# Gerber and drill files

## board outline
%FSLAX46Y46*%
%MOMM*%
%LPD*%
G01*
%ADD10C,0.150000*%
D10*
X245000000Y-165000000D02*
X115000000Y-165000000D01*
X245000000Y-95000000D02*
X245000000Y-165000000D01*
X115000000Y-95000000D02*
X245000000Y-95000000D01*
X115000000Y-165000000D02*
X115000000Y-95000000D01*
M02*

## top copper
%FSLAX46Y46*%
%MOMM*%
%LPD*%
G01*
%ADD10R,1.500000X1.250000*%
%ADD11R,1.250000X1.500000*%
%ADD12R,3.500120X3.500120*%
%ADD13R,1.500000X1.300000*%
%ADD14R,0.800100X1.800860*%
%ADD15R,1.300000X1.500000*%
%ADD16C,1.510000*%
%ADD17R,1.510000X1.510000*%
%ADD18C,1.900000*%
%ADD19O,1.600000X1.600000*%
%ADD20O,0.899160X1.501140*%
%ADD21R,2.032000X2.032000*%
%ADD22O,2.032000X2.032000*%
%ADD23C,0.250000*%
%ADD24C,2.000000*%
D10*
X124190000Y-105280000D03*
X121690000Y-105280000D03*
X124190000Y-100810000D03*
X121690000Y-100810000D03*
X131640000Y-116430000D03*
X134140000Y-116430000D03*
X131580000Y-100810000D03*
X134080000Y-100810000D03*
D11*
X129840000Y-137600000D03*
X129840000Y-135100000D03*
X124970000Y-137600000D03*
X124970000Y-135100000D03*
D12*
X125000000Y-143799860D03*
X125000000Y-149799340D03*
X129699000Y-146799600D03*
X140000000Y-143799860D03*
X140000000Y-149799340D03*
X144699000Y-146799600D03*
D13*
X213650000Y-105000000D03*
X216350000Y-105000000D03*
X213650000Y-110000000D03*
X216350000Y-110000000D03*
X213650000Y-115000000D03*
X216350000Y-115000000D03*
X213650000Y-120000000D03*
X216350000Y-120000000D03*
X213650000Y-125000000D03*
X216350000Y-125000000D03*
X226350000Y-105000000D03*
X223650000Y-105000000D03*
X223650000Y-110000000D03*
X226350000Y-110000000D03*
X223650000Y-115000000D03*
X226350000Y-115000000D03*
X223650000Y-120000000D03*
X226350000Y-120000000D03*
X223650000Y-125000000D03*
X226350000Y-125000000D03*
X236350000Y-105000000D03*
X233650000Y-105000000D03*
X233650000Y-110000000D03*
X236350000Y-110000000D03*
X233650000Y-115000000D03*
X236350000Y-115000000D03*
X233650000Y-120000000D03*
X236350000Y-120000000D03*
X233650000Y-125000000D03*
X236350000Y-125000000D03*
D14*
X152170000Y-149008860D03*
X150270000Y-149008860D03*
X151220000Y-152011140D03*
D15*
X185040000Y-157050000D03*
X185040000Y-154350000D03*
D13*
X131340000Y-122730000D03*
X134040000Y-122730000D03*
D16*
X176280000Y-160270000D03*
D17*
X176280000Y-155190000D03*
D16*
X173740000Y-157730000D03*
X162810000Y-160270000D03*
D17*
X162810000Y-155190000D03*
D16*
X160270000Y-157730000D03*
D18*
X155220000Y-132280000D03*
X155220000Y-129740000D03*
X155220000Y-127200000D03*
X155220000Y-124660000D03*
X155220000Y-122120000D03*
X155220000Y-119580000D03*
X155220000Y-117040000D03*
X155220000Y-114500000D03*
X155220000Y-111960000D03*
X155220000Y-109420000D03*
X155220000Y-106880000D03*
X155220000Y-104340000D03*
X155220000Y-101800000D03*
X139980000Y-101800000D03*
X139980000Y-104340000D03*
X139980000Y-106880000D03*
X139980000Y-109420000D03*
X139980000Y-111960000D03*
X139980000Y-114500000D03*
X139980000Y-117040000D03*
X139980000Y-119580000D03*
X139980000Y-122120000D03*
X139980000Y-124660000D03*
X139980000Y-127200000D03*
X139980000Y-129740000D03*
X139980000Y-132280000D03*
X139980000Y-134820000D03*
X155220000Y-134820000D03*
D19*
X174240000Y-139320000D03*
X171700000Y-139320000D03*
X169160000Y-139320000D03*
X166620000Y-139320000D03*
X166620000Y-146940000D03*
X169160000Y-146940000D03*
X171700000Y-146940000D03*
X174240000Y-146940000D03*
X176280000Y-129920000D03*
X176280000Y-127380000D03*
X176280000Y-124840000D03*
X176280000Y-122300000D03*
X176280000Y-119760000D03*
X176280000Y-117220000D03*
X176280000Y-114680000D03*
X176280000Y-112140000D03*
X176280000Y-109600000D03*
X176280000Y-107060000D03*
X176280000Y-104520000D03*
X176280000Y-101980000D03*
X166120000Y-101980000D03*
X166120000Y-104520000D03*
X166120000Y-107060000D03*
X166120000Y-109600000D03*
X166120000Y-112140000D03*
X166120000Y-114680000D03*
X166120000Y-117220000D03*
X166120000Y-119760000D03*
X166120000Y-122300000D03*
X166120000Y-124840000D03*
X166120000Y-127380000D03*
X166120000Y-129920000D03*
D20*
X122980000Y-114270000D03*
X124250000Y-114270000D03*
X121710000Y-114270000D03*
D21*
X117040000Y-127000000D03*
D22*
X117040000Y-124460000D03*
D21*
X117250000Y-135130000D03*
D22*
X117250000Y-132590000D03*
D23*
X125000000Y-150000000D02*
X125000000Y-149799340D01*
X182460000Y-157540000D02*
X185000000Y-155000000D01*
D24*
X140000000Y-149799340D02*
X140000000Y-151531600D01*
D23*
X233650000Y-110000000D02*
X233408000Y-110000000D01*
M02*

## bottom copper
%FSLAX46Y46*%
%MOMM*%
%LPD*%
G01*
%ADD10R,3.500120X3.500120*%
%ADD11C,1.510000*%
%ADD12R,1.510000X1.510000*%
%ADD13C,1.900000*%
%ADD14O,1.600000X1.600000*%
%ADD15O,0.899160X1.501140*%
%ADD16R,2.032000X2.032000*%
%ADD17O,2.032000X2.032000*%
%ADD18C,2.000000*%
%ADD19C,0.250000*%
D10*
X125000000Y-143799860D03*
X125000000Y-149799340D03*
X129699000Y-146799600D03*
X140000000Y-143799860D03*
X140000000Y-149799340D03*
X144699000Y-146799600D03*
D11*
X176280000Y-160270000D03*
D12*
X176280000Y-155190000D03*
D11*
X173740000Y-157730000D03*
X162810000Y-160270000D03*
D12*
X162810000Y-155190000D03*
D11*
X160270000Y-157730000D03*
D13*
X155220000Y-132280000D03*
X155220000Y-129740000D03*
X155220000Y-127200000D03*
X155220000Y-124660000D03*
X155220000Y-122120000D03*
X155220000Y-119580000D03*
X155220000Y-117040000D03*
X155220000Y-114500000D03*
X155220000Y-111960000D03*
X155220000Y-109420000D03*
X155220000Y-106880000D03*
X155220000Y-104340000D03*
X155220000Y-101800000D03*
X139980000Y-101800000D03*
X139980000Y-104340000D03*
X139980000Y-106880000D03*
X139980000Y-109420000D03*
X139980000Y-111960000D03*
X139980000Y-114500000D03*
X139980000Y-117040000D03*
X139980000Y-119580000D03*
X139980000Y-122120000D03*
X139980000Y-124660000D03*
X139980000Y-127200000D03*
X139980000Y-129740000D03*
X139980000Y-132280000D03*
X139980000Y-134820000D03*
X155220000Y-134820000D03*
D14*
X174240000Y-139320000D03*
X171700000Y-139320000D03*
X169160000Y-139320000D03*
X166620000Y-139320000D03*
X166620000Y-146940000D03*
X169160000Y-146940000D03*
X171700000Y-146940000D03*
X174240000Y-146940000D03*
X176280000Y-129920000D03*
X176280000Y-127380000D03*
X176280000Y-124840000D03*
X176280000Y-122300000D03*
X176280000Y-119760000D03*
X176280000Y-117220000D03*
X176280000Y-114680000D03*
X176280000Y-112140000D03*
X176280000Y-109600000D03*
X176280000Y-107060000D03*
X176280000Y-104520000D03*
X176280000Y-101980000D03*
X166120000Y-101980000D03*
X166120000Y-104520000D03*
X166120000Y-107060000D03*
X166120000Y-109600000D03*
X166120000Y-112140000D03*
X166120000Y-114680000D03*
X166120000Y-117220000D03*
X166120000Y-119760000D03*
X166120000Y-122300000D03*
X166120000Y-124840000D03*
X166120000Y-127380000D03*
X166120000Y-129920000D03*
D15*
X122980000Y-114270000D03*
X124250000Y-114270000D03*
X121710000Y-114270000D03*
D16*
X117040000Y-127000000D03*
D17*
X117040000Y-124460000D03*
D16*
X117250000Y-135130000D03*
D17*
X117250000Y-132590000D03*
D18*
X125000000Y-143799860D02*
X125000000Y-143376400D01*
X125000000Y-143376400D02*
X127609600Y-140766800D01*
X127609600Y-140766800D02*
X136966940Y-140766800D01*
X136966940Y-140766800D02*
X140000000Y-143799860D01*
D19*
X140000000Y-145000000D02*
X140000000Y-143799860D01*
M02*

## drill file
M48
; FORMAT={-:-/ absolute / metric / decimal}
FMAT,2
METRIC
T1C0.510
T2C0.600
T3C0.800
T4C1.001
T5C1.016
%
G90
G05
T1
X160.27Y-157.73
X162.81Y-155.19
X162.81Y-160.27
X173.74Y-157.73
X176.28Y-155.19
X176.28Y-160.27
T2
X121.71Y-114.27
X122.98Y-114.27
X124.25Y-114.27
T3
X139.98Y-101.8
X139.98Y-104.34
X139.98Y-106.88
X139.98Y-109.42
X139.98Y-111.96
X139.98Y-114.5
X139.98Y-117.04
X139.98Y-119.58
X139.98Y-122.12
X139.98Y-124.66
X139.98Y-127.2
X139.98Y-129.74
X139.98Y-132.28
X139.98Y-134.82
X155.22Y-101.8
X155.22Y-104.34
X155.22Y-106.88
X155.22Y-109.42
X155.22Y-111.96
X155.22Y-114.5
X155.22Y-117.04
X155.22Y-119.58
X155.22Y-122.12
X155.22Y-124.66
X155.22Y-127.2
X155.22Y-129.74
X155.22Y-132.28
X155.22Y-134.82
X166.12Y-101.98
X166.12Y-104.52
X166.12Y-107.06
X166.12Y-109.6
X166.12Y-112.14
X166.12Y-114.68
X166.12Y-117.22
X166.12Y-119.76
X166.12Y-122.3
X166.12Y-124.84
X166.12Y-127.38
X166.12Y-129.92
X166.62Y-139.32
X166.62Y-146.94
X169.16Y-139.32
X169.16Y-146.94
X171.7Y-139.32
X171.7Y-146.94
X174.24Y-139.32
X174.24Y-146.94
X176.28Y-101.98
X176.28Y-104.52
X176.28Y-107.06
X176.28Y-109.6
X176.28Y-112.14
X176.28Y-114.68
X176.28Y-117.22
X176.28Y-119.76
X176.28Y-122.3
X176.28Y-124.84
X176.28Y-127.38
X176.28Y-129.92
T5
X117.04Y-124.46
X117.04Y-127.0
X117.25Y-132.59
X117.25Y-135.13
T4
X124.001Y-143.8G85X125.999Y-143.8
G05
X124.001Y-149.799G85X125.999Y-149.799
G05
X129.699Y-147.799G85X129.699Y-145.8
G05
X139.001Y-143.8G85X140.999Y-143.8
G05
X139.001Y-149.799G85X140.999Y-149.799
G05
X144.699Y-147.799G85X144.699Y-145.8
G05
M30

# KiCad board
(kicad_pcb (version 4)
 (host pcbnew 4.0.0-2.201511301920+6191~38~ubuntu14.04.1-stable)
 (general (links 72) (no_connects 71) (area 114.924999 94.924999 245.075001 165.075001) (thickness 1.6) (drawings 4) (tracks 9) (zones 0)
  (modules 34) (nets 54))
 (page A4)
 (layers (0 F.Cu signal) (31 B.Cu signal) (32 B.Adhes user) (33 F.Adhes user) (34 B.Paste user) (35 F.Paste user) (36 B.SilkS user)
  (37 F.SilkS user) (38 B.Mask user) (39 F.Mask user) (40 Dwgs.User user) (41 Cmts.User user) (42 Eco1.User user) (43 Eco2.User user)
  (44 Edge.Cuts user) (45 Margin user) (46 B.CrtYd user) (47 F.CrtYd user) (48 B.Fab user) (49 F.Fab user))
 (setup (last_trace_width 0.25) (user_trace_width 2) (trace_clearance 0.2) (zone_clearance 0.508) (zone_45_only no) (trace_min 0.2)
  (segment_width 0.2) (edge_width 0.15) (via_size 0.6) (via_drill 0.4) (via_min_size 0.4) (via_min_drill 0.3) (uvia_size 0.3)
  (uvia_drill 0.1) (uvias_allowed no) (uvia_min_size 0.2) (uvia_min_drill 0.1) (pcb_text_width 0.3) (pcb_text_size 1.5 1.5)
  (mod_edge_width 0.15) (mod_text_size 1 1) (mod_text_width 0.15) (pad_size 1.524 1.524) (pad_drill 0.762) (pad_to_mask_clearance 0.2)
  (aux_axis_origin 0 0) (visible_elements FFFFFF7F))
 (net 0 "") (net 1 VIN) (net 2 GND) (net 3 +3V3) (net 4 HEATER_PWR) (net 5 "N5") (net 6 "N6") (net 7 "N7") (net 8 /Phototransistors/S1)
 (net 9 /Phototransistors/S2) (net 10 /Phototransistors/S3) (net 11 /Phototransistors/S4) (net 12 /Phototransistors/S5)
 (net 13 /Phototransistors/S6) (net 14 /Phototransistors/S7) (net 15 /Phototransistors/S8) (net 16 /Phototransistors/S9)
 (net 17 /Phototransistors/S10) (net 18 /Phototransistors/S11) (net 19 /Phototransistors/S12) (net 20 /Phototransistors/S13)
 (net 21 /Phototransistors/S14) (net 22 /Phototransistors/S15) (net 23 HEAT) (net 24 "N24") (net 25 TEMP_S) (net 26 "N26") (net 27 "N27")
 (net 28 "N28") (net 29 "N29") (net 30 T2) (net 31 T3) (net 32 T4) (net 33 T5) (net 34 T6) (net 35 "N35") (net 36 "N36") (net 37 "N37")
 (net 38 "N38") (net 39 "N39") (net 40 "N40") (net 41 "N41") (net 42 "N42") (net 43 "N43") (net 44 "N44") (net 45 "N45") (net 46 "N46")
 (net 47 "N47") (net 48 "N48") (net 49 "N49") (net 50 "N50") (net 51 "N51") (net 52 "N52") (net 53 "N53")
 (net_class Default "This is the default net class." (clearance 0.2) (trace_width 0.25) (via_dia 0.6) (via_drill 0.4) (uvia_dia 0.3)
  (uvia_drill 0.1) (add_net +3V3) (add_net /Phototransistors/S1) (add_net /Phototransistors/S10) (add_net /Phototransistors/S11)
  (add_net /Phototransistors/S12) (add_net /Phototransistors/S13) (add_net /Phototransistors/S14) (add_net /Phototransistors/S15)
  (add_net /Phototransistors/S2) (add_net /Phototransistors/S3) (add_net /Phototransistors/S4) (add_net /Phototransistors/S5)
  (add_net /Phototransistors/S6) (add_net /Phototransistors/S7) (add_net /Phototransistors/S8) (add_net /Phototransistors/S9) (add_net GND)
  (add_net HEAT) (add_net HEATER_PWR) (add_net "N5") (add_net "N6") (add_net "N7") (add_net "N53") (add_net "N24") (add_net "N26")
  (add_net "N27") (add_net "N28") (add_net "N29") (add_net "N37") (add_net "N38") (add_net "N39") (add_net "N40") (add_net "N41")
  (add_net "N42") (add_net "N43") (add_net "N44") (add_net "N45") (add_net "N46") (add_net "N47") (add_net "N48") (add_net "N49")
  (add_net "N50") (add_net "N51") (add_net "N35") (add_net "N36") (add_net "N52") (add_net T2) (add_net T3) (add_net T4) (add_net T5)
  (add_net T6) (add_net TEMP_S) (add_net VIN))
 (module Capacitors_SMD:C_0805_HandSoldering (layer F.Cu) (at 122.94 105.28 180)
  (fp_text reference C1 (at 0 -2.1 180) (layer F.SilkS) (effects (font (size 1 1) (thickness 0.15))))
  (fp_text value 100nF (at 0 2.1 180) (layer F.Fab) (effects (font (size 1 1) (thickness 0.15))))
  (pad 1 smd rect (at -1.25 0 180) (size 1.5 1.25) (layers F.Cu F.Paste F.Mask) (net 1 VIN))
  (pad 2 smd rect (at 1.25 0 180) (size 1.5 1.25) (layers F.Cu F.Paste F.Mask) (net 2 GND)))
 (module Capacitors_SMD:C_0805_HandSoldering (layer F.Cu) (at 122.94 100.81 180)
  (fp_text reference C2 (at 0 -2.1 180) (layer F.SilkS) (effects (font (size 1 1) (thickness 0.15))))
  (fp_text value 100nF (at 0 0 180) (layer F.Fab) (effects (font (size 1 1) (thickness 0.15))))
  (pad 1 smd rect (at -1.25 0 180) (size 1.5 1.25) (layers F.Cu F.Paste F.Mask) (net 1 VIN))
  (pad 2 smd rect (at 1.25 0 180) (size 1.5 1.25) (layers F.Cu F.Paste F.Mask) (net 2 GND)))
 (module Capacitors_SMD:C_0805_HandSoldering (layer F.Cu) (at 132.89 116.43)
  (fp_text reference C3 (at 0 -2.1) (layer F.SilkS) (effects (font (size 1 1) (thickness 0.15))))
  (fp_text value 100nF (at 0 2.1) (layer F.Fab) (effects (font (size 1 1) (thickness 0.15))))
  (pad 1 smd rect (at -1.25 0) (size 1.5 1.25) (layers F.Cu F.Paste F.Mask) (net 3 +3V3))
  (pad 2 smd rect (at 1.25 0) (size 1.5 1.25) (layers F.Cu F.Paste F.Mask) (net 2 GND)))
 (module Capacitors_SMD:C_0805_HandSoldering (layer F.Cu) (at 132.83 100.81)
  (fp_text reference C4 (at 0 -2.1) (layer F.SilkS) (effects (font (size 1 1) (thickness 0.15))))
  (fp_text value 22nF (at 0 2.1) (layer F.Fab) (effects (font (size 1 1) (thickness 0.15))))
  (pad 1 smd rect (at -1.25 0) (size 1.5 1.25) (layers F.Cu F.Paste F.Mask) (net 3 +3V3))
  (pad 2 smd rect (at 1.25 0) (size 1.5 1.25) (layers F.Cu F.Paste F.Mask) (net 2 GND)))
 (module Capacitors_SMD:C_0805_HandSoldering (layer F.Cu) (at 129.84 136.35 90)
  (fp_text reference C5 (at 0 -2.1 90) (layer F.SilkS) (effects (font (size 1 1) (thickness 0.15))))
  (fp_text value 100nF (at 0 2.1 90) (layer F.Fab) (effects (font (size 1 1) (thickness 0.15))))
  (pad 1 smd rect (at -1.25 0 90) (size 1.5 1.25) (layers F.Cu F.Paste F.Mask) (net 3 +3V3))
  (pad 2 smd rect (at 1.25 0 90) (size 1.5 1.25) (layers F.Cu F.Paste F.Mask) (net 2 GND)))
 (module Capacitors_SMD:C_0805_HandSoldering (layer F.Cu) (at 124.97 136.35 90)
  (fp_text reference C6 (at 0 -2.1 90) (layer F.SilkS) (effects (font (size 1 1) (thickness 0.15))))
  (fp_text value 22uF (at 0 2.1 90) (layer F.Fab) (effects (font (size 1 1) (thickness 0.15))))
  (pad 1 smd rect (at -1.25 0 90) (size 1.5 1.25) (layers F.Cu F.Paste F.Mask) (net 3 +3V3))
  (pad 2 smd rect (at 1.25 0 90) (size 1.5 1.25) (layers F.Cu F.Paste F.Mask) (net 2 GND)))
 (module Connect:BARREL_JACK (layer F.Cu) (at 125 150 90)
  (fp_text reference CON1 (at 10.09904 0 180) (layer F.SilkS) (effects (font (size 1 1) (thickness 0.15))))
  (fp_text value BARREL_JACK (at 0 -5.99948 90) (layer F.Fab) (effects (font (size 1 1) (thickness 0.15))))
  (pad 1 thru_hole rect (at 6.20014 0 90) (size 3.50012 3.50012) (drill oval 1.00076 2.99974) (layers *.Cu *.Mask F.SilkS)
   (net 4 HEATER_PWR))
  (pad 2 thru_hole rect (at 0.20066 0 90) (size 3.50012 3.50012) (drill oval 1.00076 2.99974) (layers *.Cu *.Mask F.SilkS) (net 2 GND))
  (pad 3 thru_hole rect (at 3.2004 4.699 90) (size 3.50012 3.50012) (drill oval 2.99974 1.00076) (layers *.Cu *.Mask F.SilkS) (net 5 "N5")))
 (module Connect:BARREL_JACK (layer F.Cu) (at 140 150 90)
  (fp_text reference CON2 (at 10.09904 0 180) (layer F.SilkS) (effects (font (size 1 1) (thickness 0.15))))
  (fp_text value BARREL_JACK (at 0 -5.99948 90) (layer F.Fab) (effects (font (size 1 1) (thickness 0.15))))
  (pad 1 thru_hole rect (at 6.20014 0 90) (size 3.50012 3.50012) (drill oval 1.00076 2.99974) (layers *.Cu *.Mask F.SilkS)
   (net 4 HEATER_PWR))
  (pad 2 thru_hole rect (at 0.20066 0 90) (size 3.50012 3.50012) (drill oval 1.00076 2.99974) (layers *.Cu *.Mask F.SilkS) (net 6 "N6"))
  (pad 3 thru_hole rect (at 3.2004 4.699 90) (size 3.50012 3.50012) (drill oval 2.99974 1.00076) (layers *.Cu *.Mask F.SilkS) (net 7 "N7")))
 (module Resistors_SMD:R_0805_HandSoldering (layer F.Cu) (at 215 105)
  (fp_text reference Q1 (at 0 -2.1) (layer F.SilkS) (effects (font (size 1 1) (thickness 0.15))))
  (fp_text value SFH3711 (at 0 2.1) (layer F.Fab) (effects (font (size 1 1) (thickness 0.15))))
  (pad 1 smd rect (at -1.35 0) (size 1.5 1.3) (layers F.Cu F.Paste F.Mask) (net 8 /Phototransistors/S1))
  (pad 2 smd rect (at 1.35 0) (size 1.5 1.3) (layers F.Cu F.Paste F.Mask) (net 3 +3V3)))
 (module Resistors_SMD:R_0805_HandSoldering (layer F.Cu) (at 215 110)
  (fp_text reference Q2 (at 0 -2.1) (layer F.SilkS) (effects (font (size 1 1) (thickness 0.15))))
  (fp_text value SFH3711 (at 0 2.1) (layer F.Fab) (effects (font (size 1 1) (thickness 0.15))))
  (pad 1 smd rect (at -1.35 0) (size 1.5 1.3) (layers F.Cu F.Paste F.Mask) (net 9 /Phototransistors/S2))
  (pad 2 smd rect (at 1.35 0) (size 1.5 1.3) (layers F.Cu F.Paste F.Mask) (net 3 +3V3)))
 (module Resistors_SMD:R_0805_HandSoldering (layer F.Cu) (at 215 115)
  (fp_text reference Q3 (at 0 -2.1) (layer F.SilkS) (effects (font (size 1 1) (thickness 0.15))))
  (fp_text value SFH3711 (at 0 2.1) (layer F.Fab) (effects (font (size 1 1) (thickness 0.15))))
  (pad 1 smd rect (at -1.35 0) (size 1.5 1.3) (layers F.Cu F.Paste F.Mask) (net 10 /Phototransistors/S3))
  (pad 2 smd rect (at 1.35 0) (size 1.5 1.3) (layers F.Cu F.Paste F.Mask) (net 3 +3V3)))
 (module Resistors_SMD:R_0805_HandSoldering (layer F.Cu) (at 215 120)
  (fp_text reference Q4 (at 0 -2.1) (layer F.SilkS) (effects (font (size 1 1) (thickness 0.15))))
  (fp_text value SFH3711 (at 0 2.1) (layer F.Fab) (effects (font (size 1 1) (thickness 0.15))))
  (pad 1 smd rect (at -1.35 0) (size 1.5 1.3) (layers F.Cu F.Paste F.Mask) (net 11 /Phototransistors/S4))
  (pad 2 smd rect (at 1.35 0) (size 1.5 1.3) (layers F.Cu F.Paste F.Mask) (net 3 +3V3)))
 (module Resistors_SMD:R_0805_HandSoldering (layer F.Cu) (at 215 125)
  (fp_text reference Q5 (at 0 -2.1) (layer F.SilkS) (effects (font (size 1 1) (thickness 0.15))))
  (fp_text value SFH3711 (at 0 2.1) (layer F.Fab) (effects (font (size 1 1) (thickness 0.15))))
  (pad 1 smd rect (at -1.35 0) (size 1.5 1.3) (layers F.Cu F.Paste F.Mask) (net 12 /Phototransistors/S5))
  (pad 2 smd rect (at 1.35 0) (size 1.5 1.3) (layers F.Cu F.Paste F.Mask) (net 3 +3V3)))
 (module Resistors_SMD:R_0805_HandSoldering (layer F.Cu) (at 225 105 180)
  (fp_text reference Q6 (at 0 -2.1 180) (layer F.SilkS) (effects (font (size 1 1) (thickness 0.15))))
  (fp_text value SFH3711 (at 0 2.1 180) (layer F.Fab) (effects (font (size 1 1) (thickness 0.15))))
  (pad 1 smd rect (at -1.35 0 180) (size 1.5 1.3) (layers F.Cu F.Paste F.Mask) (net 3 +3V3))
  (pad 2 smd rect (at 1.35 0 180) (size 1.5 1.3) (layers F.Cu F.Paste F.Mask) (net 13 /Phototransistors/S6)))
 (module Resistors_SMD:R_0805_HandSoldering (layer F.Cu) (at 225 110)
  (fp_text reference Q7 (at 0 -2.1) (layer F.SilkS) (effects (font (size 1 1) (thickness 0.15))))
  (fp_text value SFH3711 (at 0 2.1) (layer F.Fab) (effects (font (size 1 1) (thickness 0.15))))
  (pad 1 smd rect (at -1.35 0) (size 1.5 1.3) (layers F.Cu F.Paste F.Mask) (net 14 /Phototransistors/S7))
  (pad 2 smd rect (at 1.35 0) (size 1.5 1.3) (layers F.Cu F.Paste F.Mask) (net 3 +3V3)))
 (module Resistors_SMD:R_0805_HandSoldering (layer F.Cu) (at 225 115)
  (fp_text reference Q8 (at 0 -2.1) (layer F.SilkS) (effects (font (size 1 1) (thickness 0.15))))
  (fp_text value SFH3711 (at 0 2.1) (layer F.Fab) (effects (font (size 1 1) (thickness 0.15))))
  (pad 1 smd rect (at -1.35 0) (size 1.5 1.3) (layers F.Cu F.Paste F.Mask) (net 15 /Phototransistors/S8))
  (pad 2 smd rect (at 1.35 0) (size 1.5 1.3) (layers F.Cu F.Paste F.Mask) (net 3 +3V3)))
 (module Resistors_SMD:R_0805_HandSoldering (layer F.Cu) (at 225 120)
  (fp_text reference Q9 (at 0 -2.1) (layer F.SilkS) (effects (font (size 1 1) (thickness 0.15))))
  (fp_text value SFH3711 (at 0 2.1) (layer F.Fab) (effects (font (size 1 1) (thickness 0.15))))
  (pad 1 smd rect (at -1.35 0) (size 1.5 1.3) (layers F.Cu F.Paste F.Mask) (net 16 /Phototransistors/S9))
  (pad 2 smd rect (at 1.35 0) (size 1.5 1.3) (layers F.Cu F.Paste F.Mask) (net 3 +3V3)))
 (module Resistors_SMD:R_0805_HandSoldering (layer F.Cu) (at 225 125)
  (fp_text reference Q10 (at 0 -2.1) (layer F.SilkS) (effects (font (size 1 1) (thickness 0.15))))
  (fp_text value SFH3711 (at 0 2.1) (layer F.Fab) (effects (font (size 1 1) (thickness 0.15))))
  (pad 1 smd rect (at -1.35 0) (size 1.5 1.3) (layers F.Cu F.Paste F.Mask) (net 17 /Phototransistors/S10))
  (pad 2 smd rect (at 1.35 0) (size 1.5 1.3) (layers F.Cu F.Paste F.Mask) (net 3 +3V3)))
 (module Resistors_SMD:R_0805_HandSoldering (layer F.Cu) (at 235 105 180)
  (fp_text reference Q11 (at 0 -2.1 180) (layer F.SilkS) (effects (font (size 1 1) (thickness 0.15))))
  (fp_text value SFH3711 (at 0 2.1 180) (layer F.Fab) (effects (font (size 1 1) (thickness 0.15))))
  (pad 1 smd rect (at -1.35 0 180) (size 1.5 1.3) (layers F.Cu F.Paste F.Mask) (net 3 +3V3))
  (pad 2 smd rect (at 1.35 0 180) (size 1.5 1.3) (layers F.Cu F.Paste F.Mask) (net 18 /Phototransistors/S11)))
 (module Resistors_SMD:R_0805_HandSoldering (layer F.Cu) (at 235 110)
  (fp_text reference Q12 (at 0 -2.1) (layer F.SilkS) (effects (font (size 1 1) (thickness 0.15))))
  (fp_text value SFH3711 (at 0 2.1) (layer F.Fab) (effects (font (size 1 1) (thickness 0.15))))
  (pad 1 smd rect (at -1.35 0) (size 1.5 1.3) (layers F.Cu F.Paste F.Mask) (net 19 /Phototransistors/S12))
  (pad 2 smd rect (at 1.35 0) (size 1.5 1.3) (layers F.Cu F.Paste F.Mask) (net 3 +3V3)))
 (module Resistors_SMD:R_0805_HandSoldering (layer F.Cu) (at 235 115)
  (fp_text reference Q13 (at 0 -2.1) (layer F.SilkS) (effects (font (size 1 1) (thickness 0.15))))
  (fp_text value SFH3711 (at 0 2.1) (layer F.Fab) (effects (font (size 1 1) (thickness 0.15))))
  (pad 1 smd rect (at -1.35 0) (size 1.5 1.3) (layers F.Cu F.Paste F.Mask) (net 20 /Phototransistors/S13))
  (pad 2 smd rect (at 1.35 0) (size 1.5 1.3) (layers F.Cu F.Paste F.Mask) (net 3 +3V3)))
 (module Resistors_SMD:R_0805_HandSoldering (layer F.Cu) (at 235 120)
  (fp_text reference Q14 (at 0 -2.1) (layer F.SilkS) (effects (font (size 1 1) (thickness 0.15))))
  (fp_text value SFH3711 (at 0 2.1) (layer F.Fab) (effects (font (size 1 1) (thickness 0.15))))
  (pad 1 smd rect (at -1.35 0) (size 1.5 1.3) (layers F.Cu F.Paste F.Mask) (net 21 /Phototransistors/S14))
  (pad 2 smd rect (at 1.35 0) (size 1.5 1.3) (layers F.Cu F.Paste F.Mask) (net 3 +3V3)))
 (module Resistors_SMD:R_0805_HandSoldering (layer F.Cu) (at 235 125)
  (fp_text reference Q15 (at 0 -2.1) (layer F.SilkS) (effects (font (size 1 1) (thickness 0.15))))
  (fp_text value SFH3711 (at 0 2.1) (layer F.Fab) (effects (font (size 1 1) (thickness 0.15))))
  (pad 1 smd rect (at -1.35 0) (size 1.5 1.3) (layers F.Cu F.Paste F.Mask) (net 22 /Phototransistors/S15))
  (pad 2 smd rect (at 1.35 0) (size 1.5 1.3) (layers F.Cu F.Paste F.Mask) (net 3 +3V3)))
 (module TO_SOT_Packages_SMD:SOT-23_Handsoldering (layer F.Cu) (at 151.22 150.51 180)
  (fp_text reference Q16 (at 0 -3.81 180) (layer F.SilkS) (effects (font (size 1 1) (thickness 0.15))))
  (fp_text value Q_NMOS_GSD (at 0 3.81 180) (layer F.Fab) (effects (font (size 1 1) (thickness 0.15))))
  (pad 1 smd rect (at -0.95 1.50114 180) (size 0.8001 1.80086) (layers F.Cu F.Paste F.Mask) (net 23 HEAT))
  (pad 2 smd rect (at 0.95 1.50114 180) (size 0.8001 1.80086) (layers F.Cu F.Paste F.Mask) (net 2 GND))
  (pad 3 smd rect (at 0 -1.50114 180) (size 0.8001 1.80086) (layers F.Cu F.Paste F.Mask) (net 6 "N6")))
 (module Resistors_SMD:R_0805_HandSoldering (layer F.Cu) (at 185.04 155.7 90)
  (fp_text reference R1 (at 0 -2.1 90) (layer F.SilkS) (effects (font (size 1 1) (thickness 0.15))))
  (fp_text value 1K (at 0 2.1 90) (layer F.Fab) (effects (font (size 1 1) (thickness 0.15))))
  (pad 1 smd rect (at -1.35 0 90) (size 1.5 1.3) (layers F.Cu F.Paste F.Mask) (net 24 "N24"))
  (pad 2 smd rect (at 1.35 0 90) (size 1.5 1.3) (layers F.Cu F.Paste F.Mask) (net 2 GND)))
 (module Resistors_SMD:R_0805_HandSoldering (layer F.Cu) (at 132.69 122.73)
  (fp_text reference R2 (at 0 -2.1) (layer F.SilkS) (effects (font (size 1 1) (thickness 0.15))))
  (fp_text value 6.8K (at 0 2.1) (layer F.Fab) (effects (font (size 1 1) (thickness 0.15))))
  (pad 1 smd rect (at -1.35 0) (size 1.5 1.3) (layers F.Cu F.Paste F.Mask) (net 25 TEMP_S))
  (pad 2 smd rect (at 1.35 0) (size 1.5 1.3) (layers F.Cu F.Paste F.Mask) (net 2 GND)))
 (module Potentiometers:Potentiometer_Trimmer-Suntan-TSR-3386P (layer F.Cu) (at 176.28 155.19 270)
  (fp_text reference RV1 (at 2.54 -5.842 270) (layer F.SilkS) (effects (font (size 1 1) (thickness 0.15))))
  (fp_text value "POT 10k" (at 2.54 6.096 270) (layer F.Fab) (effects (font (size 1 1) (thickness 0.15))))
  (pad 3 thru_hole circle (at 5.08 0 270) (size 1.51 1.51) (drill 0.51) (layers *.Cu *.Mask F.SilkS) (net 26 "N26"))
  (pad 1 thru_hole rect (at 0 0 270) (size 1.51 1.51) (drill 0.51) (layers *.Cu *.Mask F.SilkS) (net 24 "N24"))
  (pad 2 thru_hole circle (at 2.54 2.54 270) (size 1.51 1.51) (drill 0.51) (layers *.Cu *.Mask F.SilkS) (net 24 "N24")))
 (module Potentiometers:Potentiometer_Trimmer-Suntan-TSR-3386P (layer F.Cu) (at 162.81 155.19 270)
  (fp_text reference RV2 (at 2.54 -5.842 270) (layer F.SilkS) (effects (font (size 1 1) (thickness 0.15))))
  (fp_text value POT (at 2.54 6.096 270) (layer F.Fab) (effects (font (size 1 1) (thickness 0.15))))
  (pad 3 thru_hole circle (at 5.08 0 270) (size 1.51 1.51) (drill 0.51) (layers *.Cu *.Mask F.SilkS) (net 2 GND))
  (pad 1 thru_hole rect (at 0 0 270) (size 1.51 1.51) (drill 0.51) (layers *.Cu *.Mask F.SilkS) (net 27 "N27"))
  (pad 2 thru_hole circle (at 2.54 2.54 270) (size 1.51 1.51) (drill 0.51) (layers *.Cu *.Mask F.SilkS) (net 27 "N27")))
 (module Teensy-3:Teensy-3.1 (layer F.Cu) (at 155.22 132.28 90)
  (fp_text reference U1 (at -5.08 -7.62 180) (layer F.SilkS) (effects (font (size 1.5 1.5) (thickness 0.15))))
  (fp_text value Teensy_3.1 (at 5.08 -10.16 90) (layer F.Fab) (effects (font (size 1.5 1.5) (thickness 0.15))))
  (pad 0 thru_hole circle (at 0 0 90) (size 1.9 1.9) (drill 0.8) (layers *.Cu *.Mask F.SilkS) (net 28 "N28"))
  (pad 1 thru_hole circle (at 2.54 0 90) (size 1.9 1.9) (drill 0.8) (layers *.Cu *.Mask F.SilkS) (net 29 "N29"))
  (pad 2 thru_hole circle (at 5.08 0 90) (size 1.9 1.9) (drill 0.8) (layers *.Cu *.Mask F.SilkS) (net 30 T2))
  (pad 3 thru_hole circle (at 7.62 0 90) (size 1.9 1.9) (drill 0.8) (layers *.Cu *.Mask F.SilkS) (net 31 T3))
  (pad 4 thru_hole circle (at 10.16 0 90) (size 1.9 1.9) (drill 0.8) (layers *.Cu *.Mask F.SilkS) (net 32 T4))
  (pad 5 thru_hole circle (at 12.7 0 90) (size 1.9 1.9) (drill 0.8) (layers *.Cu *.Mask F.SilkS) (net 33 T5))
  (pad 6 thru_hole circle (at 15.24 0 90) (size 1.9 1.9) (drill 0.8) (layers *.Cu *.Mask F.SilkS) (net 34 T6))
  (pad 7 thru_hole circle (at 17.78 0 90) (size 1.9 1.9) (drill 0.8) (layers *.Cu *.Mask F.SilkS) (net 23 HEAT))
  (pad 8 thru_hole circle (at 20.32 0 90) (size 1.9 1.9) (drill 0.8) (layers *.Cu *.Mask F.SilkS) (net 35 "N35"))
  (pad 9 thru_hole circle (at 22.86 0 90) (size 1.9 1.9) (drill 0.8) (layers *.Cu *.Mask F.SilkS) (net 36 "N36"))
  (pad 10 thru_hole circle (at 25.4 0 90) (size 1.9 1.9) (drill 0.8) (layers *.Cu *.Mask F.SilkS) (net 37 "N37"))
  (pad 11 thru_hole circle (at 27.94 0 90) (size 1.9 1.9) (drill 0.8) (layers *.Cu *.Mask F.SilkS) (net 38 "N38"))
  (pad 12 thru_hole circle (at 30.48 0 90) (size 1.9 1.9) (drill 0.8) (layers *.Cu *.Mask F.SilkS) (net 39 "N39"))
  (pad 13 thru_hole circle (at 30.48 -15.24 90) (size 1.9 1.9) (drill 0.8) (layers *.Cu *.Mask F.SilkS) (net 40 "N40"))
  (pad 14 thru_hole circle (at 27.94 -15.24 90) (size 1.9 1.9) (drill 0.8) (layers *.Cu *.Mask F.SilkS) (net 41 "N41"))
  (pad 15 thru_hole circle (at 25.4 -15.24 90) (size 1.9 1.9) (drill 0.8) (layers *.Cu *.Mask F.SilkS) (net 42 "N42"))
  (pad 16 thru_hole circle (at 22.86 -15.24 90) (size 1.9 1.9) (drill 0.8) (layers *.Cu *.Mask F.SilkS) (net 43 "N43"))
  (pad 17 thru_hole circle (at 20.32 -15.24 90) (size 1.9 1.9) (drill 0.8) (layers *.Cu *.Mask F.SilkS) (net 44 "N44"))
  (pad 18 thru_hole circle (at 17.78 -15.24 90) (size 1.9 1.9) (drill 0.8) (layers *.Cu *.Mask F.SilkS) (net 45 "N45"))
  (pad 19 thru_hole circle (at 15.24 -15.24 90) (size 1.9 1.9) (drill 0.8) (layers *.Cu *.Mask F.SilkS) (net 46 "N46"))
  (pad 20 thru_hole circle (at 12.7 -15.24 90) (size 1.9 1.9) (drill 0.8) (layers *.Cu *.Mask F.SilkS) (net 26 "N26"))
  (pad 21 thru_hole circle (at 10.16 -15.24 90) (size 1.9 1.9) (drill 0.8) (layers *.Cu *.Mask F.SilkS) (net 25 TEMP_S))
  (pad 22 thru_hole circle (at 7.62 -15.24 90) (size 1.9 1.9) (drill 0.8) (layers *.Cu *.Mask F.SilkS) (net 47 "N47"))
  (pad 23 thru_hole circle (at 5.08 -15.24 90) (size 1.9 1.9) (drill 0.8) (layers *.Cu *.Mask F.SilkS) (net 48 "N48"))
  (pad 24 thru_hole circle (at 2.54 -15.24 90) (size 1.9 1.9) (drill 0.8) (layers *.Cu *.Mask F.SilkS) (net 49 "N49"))
  (pad 25 thru_hole circle (at 0 -15.24 90) (size 1.9 1.9) (drill 0.8) (layers *.Cu *.Mask F.SilkS) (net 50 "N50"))
  (pad 26 thru_hole circle (at -2.54 -15.24 90) (size 1.9 1.9) (drill 0.8) (layers *.Cu *.Mask F.SilkS) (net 1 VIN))
  (pad 27 thru_hole circle (at -2.54 0 90) (size 1.9 1.9) (drill 0.8) (layers *.Cu *.Mask F.SilkS) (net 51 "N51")))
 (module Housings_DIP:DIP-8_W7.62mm (layer F.Cu) (at 174.24 139.32 270)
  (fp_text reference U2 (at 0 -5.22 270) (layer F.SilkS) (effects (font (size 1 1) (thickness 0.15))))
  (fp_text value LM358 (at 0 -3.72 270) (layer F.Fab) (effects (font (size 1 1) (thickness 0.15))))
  (pad 1 thru_hole oval (at 0 0 270) (size 1.6 1.6) (drill 0.8) (layers *.Cu *.Mask F.SilkS) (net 26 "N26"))
  (pad 2 thru_hole oval (at 0 2.54 270) (size 1.6 1.6) (drill 0.8) (layers *.Cu *.Mask F.SilkS) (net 24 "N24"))
  (pad 3 thru_hole oval (at 0 5.08 270) (size 1.6 1.6) (drill 0.8) (layers *.Cu *.Mask F.SilkS) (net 27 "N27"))
  (pad 4 thru_hole oval (at 0 7.62 270) (size 1.6 1.6) (drill 0.8) (layers *.Cu *.Mask F.SilkS) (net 1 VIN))
  (pad 5 thru_hole oval (at 7.62 7.62 270) (size 1.6 1.6) (drill 0.8) (layers *.Cu *.Mask F.SilkS))
  (pad 6 thru_hole oval (at 7.62 5.08 270) (size 1.6 1.6) (drill 0.8) (layers *.Cu *.Mask F.SilkS))
  (pad 7 thru_hole oval (at 7.62 2.54 270) (size 1.6 1.6) (drill 0.8) (layers *.Cu *.Mask F.SilkS))
  (pad 8 thru_hole oval (at 7.62 0 270) (size 1.6 1.6) (drill 0.8) (layers *.Cu *.Mask F.SilkS) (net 2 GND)))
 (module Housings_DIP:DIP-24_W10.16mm (layer F.Cu) (at 176.28 129.92 180)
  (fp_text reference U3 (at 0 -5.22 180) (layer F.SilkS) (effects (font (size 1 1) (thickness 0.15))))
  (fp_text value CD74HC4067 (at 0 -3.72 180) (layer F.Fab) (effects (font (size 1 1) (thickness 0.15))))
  (pad 1 thru_hole oval (at 0 0 180) (size 1.6 1.6) (drill 0.8) (layers *.Cu *.Mask F.SilkS) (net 27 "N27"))
  (pad 2 thru_hole oval (at 0 2.54 180) (size 1.6 1.6) (drill 0.8) (layers *.Cu *.Mask F.SilkS) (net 15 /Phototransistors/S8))
  (pad 3 thru_hole oval (at 0 5.08 180) (size 1.6 1.6) (drill 0.8) (layers *.Cu *.Mask F.SilkS) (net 14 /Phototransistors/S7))
  (pad 4 thru_hole oval (at 0 7.62 180) (size 1.6 1.6) (drill 0.8) (layers *.Cu *.Mask F.SilkS) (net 13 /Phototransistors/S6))
  (pad 5 thru_hole oval (at 0 10.16 180) (size 1.6 1.6) (drill 0.8) (layers *.Cu *.Mask F.SilkS) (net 12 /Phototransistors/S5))
  (pad 6 thru_hole oval (at 0 12.7 180) (size 1.6 1.6) (drill 0.8) (layers *.Cu *.Mask F.SilkS) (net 11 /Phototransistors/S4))
  (pad 7 thru_hole oval (at 0 15.24 180) (size 1.6 1.6) (drill 0.8) (layers *.Cu *.Mask F.SilkS) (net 10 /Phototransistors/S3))
  (pad 8 thru_hole oval (at 0 17.78 180) (size 1.6 1.6) (drill 0.8) (layers *.Cu *.Mask F.SilkS) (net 9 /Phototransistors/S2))
  (pad 9 thru_hole oval (at 0 20.32 180) (size 1.6 1.6) (drill 0.8) (layers *.Cu *.Mask F.SilkS) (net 8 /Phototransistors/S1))
  (pad 10 thru_hole oval (at 0 22.86 180) (size 1.6 1.6) (drill 0.8) (layers *.Cu *.Mask F.SilkS) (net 30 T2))
  (pad 11 thru_hole oval (at 0 25.4 180) (size 1.6 1.6) (drill 0.8) (layers *.Cu *.Mask F.SilkS) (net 31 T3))
  (pad 12 thru_hole oval (at 0 27.94 180) (size 1.6 1.6) (drill 0.8) (layers *.Cu *.Mask F.SilkS) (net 2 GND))
  (pad 13 thru_hole oval (at 10.16 27.94 180) (size 1.6 1.6) (drill 0.8) (layers *.Cu *.Mask F.SilkS) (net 33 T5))
  (pad 14 thru_hole oval (at 10.16 25.4 180) (size 1.6 1.6) (drill 0.8) (layers *.Cu *.Mask F.SilkS) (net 32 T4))
  (pad 15 thru_hole oval (at 10.16 22.86 180) (size 1.6 1.6) (drill 0.8) (layers *.Cu *.Mask F.SilkS) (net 34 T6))
  (pad 16 thru_hole oval (at 10.16 20.32 180) (size 1.6 1.6) (drill 0.8) (layers *.Cu *.Mask F.SilkS) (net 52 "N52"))
  (pad 17 thru_hole oval (at 10.16 17.78 180) (size 1.6 1.6) (drill 0.8) (layers *.Cu *.Mask F.SilkS) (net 22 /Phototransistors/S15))
  (pad 18 thru_hole oval (at 10.16 15.24 180) (size 1.6 1.6) (drill 0.8) (layers *.Cu *.Mask F.SilkS) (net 21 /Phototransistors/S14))
  (pad 19 thru_hole oval (at 10.16 12.7 180) (size 1.6 1.6) (drill 0.8) (layers *.Cu *.Mask F.SilkS) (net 20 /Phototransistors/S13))
  (pad 20 thru_hole oval (at 10.16 10.16 180) (size 1.6 1.6) (drill 0.8) (layers *.Cu *.Mask F.SilkS) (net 19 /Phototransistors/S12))
  (pad 21 thru_hole oval (at 10.16 7.62 180) (size 1.6 1.6) (drill 0.8) (layers *.Cu *.Mask F.SilkS) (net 18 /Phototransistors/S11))
  (pad 22 thru_hole oval (at 10.16 5.08 180) (size 1.6 1.6) (drill 0.8) (layers *.Cu *.Mask F.SilkS) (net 17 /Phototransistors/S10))
  (pad 23 thru_hole oval (at 10.16 2.54 180) (size 1.6 1.6) (drill 0.8) (layers *.Cu *.Mask F.SilkS) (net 16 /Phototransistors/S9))
  (pad 24 thru_hole oval (at 10.16 0 180) (size 1.6 1.6) (drill 0.8) (layers *.Cu *.Mask F.SilkS) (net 1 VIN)))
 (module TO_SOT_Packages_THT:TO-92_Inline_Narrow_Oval (layer F.Cu) (at 121.71 114.27)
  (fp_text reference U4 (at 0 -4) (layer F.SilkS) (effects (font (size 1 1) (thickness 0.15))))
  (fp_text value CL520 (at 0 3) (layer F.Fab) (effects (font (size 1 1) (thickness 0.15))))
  (pad 2 thru_hole oval (at 1.27 0 180) (size 0.89916 1.50114) (drill 0.6) (layers *.Cu *.Mask F.SilkS) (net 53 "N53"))
  (pad 3 thru_hole oval (at 2.54 0 180) (size 0.89916 1.50114) (drill 0.6) (layers *.Cu *.Mask F.SilkS) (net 1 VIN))
  (pad 1 thru_hole oval (at 0 0 180) (size 0.89916 1.50114) (drill 0.6) (layers *.Cu *.Mask F.SilkS) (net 2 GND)))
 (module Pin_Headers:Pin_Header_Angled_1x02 (layer F.Cu) (at 117.04 127 180)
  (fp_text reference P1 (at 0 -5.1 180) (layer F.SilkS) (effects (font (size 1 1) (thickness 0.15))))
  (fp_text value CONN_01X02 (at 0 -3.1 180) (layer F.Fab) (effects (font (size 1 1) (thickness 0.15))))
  (pad 1 thru_hole rect (at 0 0 180) (size 2.032 2.032) (drill 1.016) (layers *.Cu *.Mask F.SilkS) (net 1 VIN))
  (pad 2 thru_hole oval (at 0 2.54 180) (size 2.032 2.032) (drill 1.016) (layers *.Cu *.Mask F.SilkS) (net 25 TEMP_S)))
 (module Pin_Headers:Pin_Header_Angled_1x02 (layer F.Cu) (at 117.25 135.13 180)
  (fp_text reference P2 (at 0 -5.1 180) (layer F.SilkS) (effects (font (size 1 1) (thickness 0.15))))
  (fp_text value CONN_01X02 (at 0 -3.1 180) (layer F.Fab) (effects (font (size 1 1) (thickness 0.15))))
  (pad 1 thru_hole rect (at 0 0 180) (size 2.032 2.032) (drill 1.016) (layers *.Cu *.Mask F.SilkS) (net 2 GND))
  (pad 2 thru_hole oval (at 0 2.54 180) (size 2.032 2.032) (drill 1.016) (layers *.Cu *.Mask F.SilkS) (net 53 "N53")))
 (gr_line (start 245 165) (end 115 165) (angle 90) (layer Edge.Cuts) (width 0.15))
 (gr_line (start 245 95) (end 245 165) (angle 90) (layer Edge.Cuts) (width 0.15))
 (gr_line (start 115 95) (end 245 95) (angle 90) (layer Edge.Cuts) (width 0.15))
 (gr_line (start 115 165) (end 115 95) (angle 90) (layer Edge.Cuts) (width 0.15))
 (segment (start 125 150) (end 125 149.79934) (width 0.25) (layer F.Cu) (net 2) (status 80000))
 (segment (start 182.46 157.54) (end 185 155) (width 0.25) (layer F.Cu) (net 2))
 (segment (start 125 143.79986) (end 125 143.3764) (width 2) (layer B.Cu) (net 4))
 (segment (start 125 143.3764) (end 127.6096 140.7668) (width 2) (layer B.Cu) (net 4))
 (segment (start 127.6096 140.7668) (end 136.96694 140.7668) (width 2) (layer B.Cu) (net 4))
 (segment (start 136.96694 140.7668) (end 140 143.79986) (width 2) (layer B.Cu) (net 4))
 (segment (start 140 145) (end 140 143.79986) (width 0.25) (layer B.Cu) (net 4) (status 80000))
 (segment (start 140 149.79934) (end 140 151.5316) (width 2) (layer F.Cu) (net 6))
 (segment (start 233.65 110) (end 233.408 110) (width 0.25) (layer F.Cu) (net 19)))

